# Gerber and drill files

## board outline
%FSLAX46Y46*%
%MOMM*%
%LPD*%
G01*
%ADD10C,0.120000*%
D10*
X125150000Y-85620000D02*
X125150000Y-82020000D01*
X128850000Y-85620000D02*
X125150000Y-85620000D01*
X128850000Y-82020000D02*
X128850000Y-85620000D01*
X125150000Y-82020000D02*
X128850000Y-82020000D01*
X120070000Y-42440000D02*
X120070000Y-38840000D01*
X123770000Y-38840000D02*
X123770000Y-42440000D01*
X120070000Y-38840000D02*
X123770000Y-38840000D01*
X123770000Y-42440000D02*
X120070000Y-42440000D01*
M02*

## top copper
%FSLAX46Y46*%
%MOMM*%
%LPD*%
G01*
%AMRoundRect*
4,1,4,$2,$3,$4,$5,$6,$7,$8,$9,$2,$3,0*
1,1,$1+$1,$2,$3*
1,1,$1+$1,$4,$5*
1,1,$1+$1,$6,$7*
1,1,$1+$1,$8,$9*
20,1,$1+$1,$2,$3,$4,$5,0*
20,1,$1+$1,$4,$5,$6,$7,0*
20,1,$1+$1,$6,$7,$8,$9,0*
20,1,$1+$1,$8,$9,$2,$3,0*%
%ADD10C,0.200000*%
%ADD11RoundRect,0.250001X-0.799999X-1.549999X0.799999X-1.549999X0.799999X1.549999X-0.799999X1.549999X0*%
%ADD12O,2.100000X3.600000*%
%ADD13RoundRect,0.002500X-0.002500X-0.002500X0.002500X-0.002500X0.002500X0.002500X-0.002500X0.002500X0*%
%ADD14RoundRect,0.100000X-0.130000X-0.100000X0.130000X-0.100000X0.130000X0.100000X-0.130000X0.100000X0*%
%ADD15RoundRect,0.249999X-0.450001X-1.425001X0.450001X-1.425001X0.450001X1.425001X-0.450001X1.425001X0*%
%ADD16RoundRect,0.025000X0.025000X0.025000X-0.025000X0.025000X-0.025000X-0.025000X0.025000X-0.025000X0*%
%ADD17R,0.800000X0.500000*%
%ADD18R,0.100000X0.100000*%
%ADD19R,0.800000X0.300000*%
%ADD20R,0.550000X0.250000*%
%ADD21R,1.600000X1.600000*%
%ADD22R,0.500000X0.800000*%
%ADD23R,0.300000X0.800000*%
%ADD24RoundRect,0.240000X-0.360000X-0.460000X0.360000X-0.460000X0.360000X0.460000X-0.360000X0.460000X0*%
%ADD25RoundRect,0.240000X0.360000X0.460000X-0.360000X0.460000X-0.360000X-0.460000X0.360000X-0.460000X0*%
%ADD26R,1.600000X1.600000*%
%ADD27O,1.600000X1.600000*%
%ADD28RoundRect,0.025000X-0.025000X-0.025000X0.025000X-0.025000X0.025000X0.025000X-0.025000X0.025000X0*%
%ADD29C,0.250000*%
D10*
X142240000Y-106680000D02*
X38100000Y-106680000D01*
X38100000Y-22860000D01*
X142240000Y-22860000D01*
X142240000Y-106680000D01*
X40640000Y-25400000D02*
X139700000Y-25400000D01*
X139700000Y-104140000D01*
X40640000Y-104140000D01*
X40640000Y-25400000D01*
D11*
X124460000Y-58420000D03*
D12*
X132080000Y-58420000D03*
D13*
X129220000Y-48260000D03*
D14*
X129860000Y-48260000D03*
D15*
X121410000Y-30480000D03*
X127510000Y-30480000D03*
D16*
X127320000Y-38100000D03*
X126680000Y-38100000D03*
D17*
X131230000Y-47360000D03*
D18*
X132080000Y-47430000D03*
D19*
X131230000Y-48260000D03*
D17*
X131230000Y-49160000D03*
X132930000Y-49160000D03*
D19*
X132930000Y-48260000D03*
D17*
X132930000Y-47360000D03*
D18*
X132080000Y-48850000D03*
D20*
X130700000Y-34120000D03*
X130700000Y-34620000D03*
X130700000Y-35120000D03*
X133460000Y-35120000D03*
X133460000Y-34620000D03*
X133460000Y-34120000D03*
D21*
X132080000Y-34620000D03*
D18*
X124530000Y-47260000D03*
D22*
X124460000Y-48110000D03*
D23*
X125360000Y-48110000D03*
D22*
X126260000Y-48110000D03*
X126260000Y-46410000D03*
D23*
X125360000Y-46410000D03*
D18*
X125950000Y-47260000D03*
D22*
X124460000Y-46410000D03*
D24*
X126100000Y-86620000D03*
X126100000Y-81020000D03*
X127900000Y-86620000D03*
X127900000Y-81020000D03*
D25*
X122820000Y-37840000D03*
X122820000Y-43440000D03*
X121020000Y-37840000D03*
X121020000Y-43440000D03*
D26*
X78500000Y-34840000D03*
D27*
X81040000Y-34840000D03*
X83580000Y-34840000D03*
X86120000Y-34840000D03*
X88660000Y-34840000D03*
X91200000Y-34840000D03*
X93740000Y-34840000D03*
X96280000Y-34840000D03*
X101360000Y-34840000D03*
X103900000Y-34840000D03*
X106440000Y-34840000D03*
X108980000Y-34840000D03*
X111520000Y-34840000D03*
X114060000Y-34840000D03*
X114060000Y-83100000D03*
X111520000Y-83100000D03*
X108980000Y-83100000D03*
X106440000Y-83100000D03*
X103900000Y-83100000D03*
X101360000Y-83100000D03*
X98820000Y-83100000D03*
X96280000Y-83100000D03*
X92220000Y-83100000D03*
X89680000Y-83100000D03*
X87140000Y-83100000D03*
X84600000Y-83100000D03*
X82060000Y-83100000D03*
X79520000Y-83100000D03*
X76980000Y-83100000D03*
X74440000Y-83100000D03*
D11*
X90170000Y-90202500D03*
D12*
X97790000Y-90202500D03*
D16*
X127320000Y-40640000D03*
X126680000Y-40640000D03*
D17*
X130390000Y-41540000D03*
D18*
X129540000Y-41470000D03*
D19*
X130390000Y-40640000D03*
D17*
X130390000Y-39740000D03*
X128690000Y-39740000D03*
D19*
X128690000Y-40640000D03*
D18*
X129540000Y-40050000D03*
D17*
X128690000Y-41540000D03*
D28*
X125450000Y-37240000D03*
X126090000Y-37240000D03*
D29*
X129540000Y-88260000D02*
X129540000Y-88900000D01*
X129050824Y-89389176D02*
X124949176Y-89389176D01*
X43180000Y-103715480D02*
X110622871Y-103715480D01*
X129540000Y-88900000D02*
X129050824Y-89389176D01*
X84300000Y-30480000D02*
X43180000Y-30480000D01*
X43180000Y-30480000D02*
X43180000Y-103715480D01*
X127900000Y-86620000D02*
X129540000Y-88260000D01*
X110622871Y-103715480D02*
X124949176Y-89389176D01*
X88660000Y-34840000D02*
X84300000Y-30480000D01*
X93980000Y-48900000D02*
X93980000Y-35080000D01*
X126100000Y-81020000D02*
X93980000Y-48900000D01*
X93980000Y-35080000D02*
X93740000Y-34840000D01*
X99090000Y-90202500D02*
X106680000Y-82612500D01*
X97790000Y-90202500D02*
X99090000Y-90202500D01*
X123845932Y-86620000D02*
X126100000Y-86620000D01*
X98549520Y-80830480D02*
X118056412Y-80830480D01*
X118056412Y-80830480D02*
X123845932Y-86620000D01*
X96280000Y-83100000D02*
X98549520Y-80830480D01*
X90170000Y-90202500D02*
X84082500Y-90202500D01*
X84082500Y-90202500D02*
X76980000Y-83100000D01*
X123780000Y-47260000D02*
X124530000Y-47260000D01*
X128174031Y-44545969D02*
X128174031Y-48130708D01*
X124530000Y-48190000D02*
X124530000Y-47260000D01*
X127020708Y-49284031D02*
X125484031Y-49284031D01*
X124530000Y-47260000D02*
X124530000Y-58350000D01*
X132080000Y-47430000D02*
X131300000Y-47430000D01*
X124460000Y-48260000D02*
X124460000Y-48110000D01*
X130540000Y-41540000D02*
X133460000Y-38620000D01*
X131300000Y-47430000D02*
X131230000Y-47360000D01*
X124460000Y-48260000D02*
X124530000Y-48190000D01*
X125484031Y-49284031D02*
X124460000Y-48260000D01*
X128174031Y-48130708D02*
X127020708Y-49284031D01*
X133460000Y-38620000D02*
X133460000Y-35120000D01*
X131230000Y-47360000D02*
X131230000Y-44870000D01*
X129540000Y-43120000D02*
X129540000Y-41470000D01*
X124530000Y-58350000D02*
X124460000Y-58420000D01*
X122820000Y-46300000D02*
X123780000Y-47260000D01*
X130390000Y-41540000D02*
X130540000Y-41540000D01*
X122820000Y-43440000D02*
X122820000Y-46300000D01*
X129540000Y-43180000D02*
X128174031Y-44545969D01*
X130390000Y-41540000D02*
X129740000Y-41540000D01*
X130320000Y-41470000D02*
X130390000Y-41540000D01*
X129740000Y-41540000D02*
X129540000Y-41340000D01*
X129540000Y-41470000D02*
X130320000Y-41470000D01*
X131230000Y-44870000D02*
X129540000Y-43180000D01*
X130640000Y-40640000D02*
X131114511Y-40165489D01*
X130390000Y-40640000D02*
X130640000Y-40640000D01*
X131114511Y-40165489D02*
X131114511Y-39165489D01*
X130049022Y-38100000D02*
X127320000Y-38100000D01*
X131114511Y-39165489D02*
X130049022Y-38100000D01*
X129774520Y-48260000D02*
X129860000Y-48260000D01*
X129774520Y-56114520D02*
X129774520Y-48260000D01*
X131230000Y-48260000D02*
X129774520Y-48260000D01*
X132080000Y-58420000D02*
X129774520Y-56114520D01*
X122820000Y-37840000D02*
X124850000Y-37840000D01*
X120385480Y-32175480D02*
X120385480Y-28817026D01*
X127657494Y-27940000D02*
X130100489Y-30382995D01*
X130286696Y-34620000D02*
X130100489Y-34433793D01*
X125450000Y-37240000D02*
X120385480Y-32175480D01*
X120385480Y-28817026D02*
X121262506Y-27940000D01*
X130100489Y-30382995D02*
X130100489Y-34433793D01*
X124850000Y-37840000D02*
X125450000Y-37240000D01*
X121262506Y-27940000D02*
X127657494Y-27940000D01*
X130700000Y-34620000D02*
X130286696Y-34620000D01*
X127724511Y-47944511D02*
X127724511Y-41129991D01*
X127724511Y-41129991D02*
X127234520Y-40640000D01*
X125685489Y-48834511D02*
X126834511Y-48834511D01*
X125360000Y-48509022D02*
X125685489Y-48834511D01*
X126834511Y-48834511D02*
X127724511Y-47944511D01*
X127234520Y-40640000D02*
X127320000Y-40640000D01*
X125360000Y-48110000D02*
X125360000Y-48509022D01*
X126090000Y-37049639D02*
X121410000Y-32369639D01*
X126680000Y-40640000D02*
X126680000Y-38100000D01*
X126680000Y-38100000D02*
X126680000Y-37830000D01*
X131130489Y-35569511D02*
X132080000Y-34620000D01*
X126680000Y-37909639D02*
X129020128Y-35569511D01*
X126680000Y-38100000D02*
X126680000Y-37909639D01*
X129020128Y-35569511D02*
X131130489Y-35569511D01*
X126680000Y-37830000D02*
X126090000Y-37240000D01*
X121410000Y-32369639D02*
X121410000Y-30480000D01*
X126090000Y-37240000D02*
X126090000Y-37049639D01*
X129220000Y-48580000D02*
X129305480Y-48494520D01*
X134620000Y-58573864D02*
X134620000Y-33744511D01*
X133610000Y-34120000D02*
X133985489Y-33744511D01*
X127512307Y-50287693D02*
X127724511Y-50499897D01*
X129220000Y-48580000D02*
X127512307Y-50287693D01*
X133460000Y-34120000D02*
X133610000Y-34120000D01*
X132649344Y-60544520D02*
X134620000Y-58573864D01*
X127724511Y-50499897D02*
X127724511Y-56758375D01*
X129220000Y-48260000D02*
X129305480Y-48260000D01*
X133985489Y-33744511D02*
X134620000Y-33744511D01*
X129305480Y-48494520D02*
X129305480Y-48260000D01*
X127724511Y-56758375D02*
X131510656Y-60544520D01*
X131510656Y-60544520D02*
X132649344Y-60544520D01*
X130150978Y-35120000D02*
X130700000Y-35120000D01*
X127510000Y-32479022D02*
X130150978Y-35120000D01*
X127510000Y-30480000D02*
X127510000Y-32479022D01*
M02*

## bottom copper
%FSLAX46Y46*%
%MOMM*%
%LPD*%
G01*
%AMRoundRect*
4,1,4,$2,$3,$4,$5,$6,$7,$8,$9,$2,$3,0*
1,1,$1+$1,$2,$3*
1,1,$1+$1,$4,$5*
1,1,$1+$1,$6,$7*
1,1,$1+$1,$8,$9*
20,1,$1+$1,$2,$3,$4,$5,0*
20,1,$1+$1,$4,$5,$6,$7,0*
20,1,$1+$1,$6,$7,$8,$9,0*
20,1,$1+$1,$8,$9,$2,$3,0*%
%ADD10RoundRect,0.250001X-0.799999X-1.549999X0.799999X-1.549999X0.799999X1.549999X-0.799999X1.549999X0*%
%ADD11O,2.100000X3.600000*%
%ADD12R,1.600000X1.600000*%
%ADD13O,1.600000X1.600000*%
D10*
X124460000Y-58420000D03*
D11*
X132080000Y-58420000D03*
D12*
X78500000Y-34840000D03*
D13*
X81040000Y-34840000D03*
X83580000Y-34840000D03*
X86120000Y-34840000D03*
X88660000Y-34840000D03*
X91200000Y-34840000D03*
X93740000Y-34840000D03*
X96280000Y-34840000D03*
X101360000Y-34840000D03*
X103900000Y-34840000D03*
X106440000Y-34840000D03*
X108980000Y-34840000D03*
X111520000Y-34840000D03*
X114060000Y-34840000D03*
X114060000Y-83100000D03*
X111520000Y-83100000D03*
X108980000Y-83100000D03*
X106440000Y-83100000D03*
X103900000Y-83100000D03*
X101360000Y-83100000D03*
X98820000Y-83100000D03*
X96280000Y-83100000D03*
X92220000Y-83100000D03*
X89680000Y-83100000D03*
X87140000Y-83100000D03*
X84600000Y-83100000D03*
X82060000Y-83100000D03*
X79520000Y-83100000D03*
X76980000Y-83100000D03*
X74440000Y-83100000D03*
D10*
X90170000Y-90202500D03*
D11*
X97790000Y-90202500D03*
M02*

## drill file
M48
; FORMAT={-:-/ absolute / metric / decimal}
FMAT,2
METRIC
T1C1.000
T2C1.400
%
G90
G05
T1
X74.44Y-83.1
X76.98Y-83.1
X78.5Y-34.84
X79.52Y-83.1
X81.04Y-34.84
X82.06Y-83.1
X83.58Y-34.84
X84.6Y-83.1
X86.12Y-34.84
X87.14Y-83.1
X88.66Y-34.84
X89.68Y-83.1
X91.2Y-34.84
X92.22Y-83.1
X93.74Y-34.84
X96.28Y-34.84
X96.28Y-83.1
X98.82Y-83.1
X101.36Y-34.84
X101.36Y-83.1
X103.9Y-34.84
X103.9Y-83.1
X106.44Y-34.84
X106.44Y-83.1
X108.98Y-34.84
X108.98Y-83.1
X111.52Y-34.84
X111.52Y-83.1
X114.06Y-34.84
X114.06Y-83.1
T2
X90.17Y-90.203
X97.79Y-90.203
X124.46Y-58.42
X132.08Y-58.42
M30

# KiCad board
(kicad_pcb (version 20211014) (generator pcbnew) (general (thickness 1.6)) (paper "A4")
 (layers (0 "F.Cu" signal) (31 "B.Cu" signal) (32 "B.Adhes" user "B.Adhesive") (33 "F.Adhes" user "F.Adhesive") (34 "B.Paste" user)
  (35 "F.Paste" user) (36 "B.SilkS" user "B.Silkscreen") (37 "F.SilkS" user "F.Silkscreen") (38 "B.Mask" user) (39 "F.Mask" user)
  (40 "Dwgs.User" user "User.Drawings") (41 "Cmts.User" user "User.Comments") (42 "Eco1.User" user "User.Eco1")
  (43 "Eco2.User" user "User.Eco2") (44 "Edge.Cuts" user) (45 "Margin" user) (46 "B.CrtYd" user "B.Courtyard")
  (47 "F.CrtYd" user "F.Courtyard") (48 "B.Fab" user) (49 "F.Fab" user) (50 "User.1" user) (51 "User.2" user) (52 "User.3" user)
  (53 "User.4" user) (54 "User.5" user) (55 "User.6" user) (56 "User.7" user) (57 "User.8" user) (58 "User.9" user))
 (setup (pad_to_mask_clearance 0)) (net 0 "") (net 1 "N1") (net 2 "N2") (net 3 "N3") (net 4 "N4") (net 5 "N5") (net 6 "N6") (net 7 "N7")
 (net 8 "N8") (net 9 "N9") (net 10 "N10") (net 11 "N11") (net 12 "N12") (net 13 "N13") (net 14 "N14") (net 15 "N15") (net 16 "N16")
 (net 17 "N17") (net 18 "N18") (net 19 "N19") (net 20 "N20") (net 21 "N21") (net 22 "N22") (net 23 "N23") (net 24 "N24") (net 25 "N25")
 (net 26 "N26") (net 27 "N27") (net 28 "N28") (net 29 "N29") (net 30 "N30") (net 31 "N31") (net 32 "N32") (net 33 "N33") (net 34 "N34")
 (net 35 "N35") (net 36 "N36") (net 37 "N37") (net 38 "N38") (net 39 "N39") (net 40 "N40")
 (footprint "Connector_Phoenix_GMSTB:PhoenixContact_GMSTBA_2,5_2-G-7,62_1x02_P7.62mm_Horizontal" (layer "F.Cu") (at 124.46 58.42)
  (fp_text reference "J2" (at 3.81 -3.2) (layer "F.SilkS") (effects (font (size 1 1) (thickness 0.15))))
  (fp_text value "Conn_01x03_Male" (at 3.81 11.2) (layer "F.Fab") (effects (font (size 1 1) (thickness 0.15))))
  (pad "1" thru_hole roundrect (at 0 0) (size 2.1 3.6) (drill 1.4) (layers *.Cu *.Mask) (roundrect_rratio 0.119048) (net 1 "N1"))
  (pad "2" thru_hole oval (at 7.62 0) (size 2.1 3.6) (drill 1.4) (layers *.Cu *.Mask) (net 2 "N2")))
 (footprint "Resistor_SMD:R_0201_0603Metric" (layer "F.Cu") (at 129.54 48.26)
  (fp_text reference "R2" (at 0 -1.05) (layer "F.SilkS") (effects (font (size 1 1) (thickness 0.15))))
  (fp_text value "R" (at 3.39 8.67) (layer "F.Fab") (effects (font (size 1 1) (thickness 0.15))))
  (pad "" smd roundrect (at -0.345 0) (size 0.318 0.36) (layers "F.Paste") (roundrect_rratio 0.25))
  (pad "" smd roundrect (at 0.345 0) (size 0.318 0.36) (layers "F.Paste") (roundrect_rratio 0.25))
  (pad "1" smd roundrect (at -0.32 0) (size 0.01 0.01) (layers "F.Cu" "F.Mask") (roundrect_rratio 0.25) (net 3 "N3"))
  (pad "2" smd roundrect (at 0.32 0) (size 0.46 0.4) (layers "F.Cu" "F.Mask") (roundrect_rratio 0.25) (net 2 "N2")))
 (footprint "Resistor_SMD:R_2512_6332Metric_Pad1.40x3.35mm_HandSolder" (layer "F.Cu") (at 124.46 30.48)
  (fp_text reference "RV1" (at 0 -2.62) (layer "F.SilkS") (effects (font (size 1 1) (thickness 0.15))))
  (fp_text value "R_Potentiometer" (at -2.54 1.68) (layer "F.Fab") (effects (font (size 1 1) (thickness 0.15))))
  (pad "1" smd roundrect (at -3.05 0) (size 1.4 3.35) (layers "F.Cu" "F.Paste" "F.Mask") (roundrect_rratio 0.178571) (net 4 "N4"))
  (pad "2" smd roundrect (at 3.05 0) (size 1.4 3.35) (layers "F.Cu" "F.Paste" "F.Mask") (roundrect_rratio 0.178571) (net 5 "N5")))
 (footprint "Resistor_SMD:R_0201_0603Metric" (layer "F.Cu") (at 127 38.1 180)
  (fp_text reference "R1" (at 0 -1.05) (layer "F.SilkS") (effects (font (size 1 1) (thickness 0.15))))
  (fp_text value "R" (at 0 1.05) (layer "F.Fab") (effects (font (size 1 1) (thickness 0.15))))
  (pad "" smd roundrect (at -0.345 0 180) (size 0.318 0.36) (layers "F.Paste") (roundrect_rratio 0.25))
  (pad "" smd roundrect (at 0.345 0 180) (size 0.1 0.1) (layers "F.Paste") (roundrect_rratio 0.25))
  (pad "1" smd roundrect (at -0.32 0 180) (size 0.1 0.1) (layers "F.Cu" "F.Mask") (roundrect_rratio 0.25) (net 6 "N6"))
  (pad "2" smd roundrect (at 0.32 0 180) (size 0.1 0.1) (layers "F.Cu" "F.Mask") (roundrect_rratio 0.25) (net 4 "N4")))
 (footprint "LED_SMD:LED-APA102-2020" (layer "F.Cu") (at 132.08 48.26)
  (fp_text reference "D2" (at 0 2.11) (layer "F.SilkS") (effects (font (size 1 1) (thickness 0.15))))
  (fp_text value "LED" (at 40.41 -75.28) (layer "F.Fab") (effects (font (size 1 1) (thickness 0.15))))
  (pad "1" smd rect (at -0.85 -0.9) (size 0.8 0.5) (layers "F.Cu" "F.Paste" "F.Mask") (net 1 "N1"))
  (pad "1" smd rect (at 0 -0.83 90) (size 0.1 0.1) (layers "F.Cu" "F.Paste" "F.Mask") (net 1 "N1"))
  (pad "2" smd rect (at -0.85 0) (size 0.8 0.3) (layers "F.Cu" "F.Paste" "F.Mask") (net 2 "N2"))
  (pad "3" smd rect (at -0.85 0.9) (size 0.8 0.5) (layers "F.Cu" "F.Paste" "F.Mask"))
  (pad "4" smd rect (at 0.85 0.9) (size 0.8 0.5) (layers "F.Cu" "F.Paste" "F.Mask"))
  (pad "5" smd rect (at 0.85 0) (size 0.8 0.3) (layers "F.Cu" "F.Paste" "F.Mask"))
  (pad "6" smd rect (at 0.85 -0.9) (size 0.8 0.5) (layers "F.Cu" "F.Paste" "F.Mask"))
  (pad "6" smd rect (at 0 0.59 90) (size 0.1 0.1) (layers "F.Cu" "F.Paste" "F.Mask")))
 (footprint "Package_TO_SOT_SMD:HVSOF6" (layer "F.Cu") (at 132.08 34.62)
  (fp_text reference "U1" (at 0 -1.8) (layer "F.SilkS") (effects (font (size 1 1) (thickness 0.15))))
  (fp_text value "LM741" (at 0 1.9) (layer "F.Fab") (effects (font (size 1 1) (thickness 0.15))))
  (pad "1" smd rect (at -1.38 -0.5 270) (size 0.25 0.55) (layers "F.Cu" "F.Paste" "F.Mask") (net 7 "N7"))
  (pad "2" smd rect (at -1.38 0 270) (size 0.25 0.55) (layers "F.Cu" "F.Paste" "F.Mask") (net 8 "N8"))
  (pad "3" smd rect (at -1.38 0.5 270) (size 0.25 0.55) (layers "F.Cu" "F.Paste" "F.Mask") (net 5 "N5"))
  (pad "4" smd rect (at 1.38 0.5 270) (size 0.25 0.55) (layers "F.Cu" "F.Paste" "F.Mask") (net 1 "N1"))
  (pad "5" smd rect (at 1.38 0 270) (size 0.25 0.55) (layers "F.Cu" "F.Paste" "F.Mask") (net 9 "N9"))
  (pad "6" smd rect (at 1.38 -0.5 270) (size 0.25 0.55) (layers "F.Cu" "F.Paste" "F.Mask") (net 3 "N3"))
  (pad "7" smd rect (at 0 0) (size 1.6 1.6) (layers "F.Cu" "F.Paste" "F.Mask") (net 4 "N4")))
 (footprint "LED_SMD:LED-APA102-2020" (layer "F.Cu") (at 125.36 47.26 90)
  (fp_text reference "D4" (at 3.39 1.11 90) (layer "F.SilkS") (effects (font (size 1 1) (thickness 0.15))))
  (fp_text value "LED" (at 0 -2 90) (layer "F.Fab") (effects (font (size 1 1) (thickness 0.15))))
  (pad "1" smd rect (at 0 -0.83 180) (size 0.1 0.1) (layers "F.Cu" "F.Paste" "F.Mask") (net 1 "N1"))
  (pad "1" smd rect (at -0.85 -0.9 90) (size 0.8 0.5) (layers "F.Cu" "F.Paste" "F.Mask") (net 1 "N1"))
  (pad "2" smd rect (at -0.85 0 90) (size 0.8 0.3) (layers "F.Cu" "F.Paste" "F.Mask") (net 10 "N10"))
  (pad "3" smd rect (at -0.85 0.9 90) (size 0.8 0.5) (layers "F.Cu" "F.Paste" "F.Mask"))
  (pad "4" smd rect (at 0.85 0.9 90) (size 0.8 0.5) (layers "F.Cu" "F.Paste" "F.Mask"))
  (pad "5" smd rect (at 0.85 0 90) (size 0.8 0.3) (layers "F.Cu" "F.Paste" "F.Mask"))
  (pad "6" smd rect (at 0 0.59 180) (size 0.1 0.1) (layers "F.Cu" "F.Paste" "F.Mask"))
  (pad "6" smd rect (at 0.85 -0.9 90) (size 0.8 0.5) (layers "F.Cu" "F.Paste" "F.Mask")))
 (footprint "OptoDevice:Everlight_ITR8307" (layer "F.Cu") (at 127 83.82)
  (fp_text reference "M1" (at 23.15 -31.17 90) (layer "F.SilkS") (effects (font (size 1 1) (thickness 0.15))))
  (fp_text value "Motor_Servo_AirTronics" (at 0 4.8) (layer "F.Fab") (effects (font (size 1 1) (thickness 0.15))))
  (fp_line (start -1.85 1.8) (end -1.85 -1.8) (layer "Edge.Cuts") (width 0.12))
  (fp_line (start 1.85 1.8) (end -1.85 1.8) (layer "Edge.Cuts") (width 0.12))
  (fp_line (start 1.85 -1.8) (end 1.85 1.8) (layer "Edge.Cuts") (width 0.12))
  (fp_line (start -1.85 -1.8) (end 1.85 -1.8) (layer "Edge.Cuts") (width 0.12))
  (pad "1" smd roundrect (at -0.9 2.8) (size 1.2 1.4) (layers "F.Cu" "F.Paste" "F.Mask") (roundrect_rratio 0.2) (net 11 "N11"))
  (pad "2" smd roundrect (at -0.9 -2.8) (size 1.2 1.4) (layers "F.Cu" "F.Paste" "F.Mask") (roundrect_rratio 0.2) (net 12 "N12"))
  (pad "3" smd roundrect (at 0.9 2.8) (size 1.2 1.4) (layers "F.Cu" "F.Paste" "F.Mask") (roundrect_rratio 0.2) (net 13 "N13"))
  (pad "4" smd roundrect (at 0.9 -2.8) (size 1.2 1.4) (layers "F.Cu" "F.Paste" "F.Mask") (roundrect_rratio 0.2)))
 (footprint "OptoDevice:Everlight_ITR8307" (layer "F.Cu") (at 121.92 40.64 180)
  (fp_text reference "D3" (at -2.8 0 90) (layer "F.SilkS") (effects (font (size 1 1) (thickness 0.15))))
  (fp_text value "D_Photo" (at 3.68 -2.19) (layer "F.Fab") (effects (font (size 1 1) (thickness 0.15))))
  (fp_line (start 1.85 -1.8) (end 1.85 1.8) (layer "Edge.Cuts") (width 0.12))
  (fp_line (start -1.85 1.8) (end -1.85 -1.8) (layer "Edge.Cuts") (width 0.12))
  (fp_line (start 1.85 1.8) (end -1.85 1.8) (layer "Edge.Cuts") (width 0.12))
  (fp_line (start -1.85 -1.8) (end 1.85 -1.8) (layer "Edge.Cuts") (width 0.12))
  (pad "1" smd roundrect (at -0.9 2.8 180) (size 1.2 1.4) (layers "F.Cu" "F.Paste" "F.Mask") (roundrect_rratio 0.2) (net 8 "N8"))
  (pad "2" smd roundrect (at -0.9 -2.8 180) (size 1.2 1.4) (layers "F.Cu" "F.Paste" "F.Mask") (roundrect_rratio 0.2) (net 1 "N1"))
  (pad "3" smd roundrect (at 0.9 2.8 180) (size 1.2 1.4) (layers "F.Cu" "F.Paste" "F.Mask") (roundrect_rratio 0.2))
  (pad "4" smd roundrect (at 0.9 -2.8 180) (size 1.2 1.4) (layers "F.Cu" "F.Paste" "F.Mask") (roundrect_rratio 0.2)))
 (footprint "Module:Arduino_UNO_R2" (layer "F.Cu") (at 78.5 34.84)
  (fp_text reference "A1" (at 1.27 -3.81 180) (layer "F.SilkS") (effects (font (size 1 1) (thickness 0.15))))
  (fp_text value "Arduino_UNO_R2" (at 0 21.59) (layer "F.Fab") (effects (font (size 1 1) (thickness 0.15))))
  (pad "1" thru_hole rect (at 0 0 90) (size 1.6 1.6) (drill 1) (layers *.Cu *.Mask) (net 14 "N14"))
  (pad "2" thru_hole oval (at 2.54 0 90) (size 1.6 1.6) (drill 1) (layers *.Cu *.Mask) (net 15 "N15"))
  (pad "3" thru_hole oval (at 5.08 0 90) (size 1.6 1.6) (drill 1) (layers *.Cu *.Mask) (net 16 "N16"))
  (pad "4" thru_hole oval (at 7.62 0 90) (size 1.6 1.6) (drill 1) (layers *.Cu *.Mask) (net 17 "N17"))
  (pad "5" thru_hole oval (at 10.16 0 90) (size 1.6 1.6) (drill 1) (layers *.Cu *.Mask) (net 13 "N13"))
  (pad "6" thru_hole oval (at 12.7 0 90) (size 1.6 1.6) (drill 1) (layers *.Cu *.Mask) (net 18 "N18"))
  (pad "7" thru_hole oval (at 15.24 0 90) (size 1.6 1.6) (drill 1) (layers *.Cu *.Mask) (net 12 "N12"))
  (pad "8" thru_hole oval (at 17.78 0 90) (size 1.6 1.6) (drill 1) (layers *.Cu *.Mask) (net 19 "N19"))
  (pad "9" thru_hole oval (at 22.86 0 90) (size 1.6 1.6) (drill 1) (layers *.Cu *.Mask) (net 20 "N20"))
  (pad "10" thru_hole oval (at 25.4 0 90) (size 1.6 1.6) (drill 1) (layers *.Cu *.Mask) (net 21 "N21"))
  (pad "11" thru_hole oval (at 27.94 0 90) (size 1.6 1.6) (drill 1) (layers *.Cu *.Mask) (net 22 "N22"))
  (pad "12" thru_hole oval (at 30.48 0 90) (size 1.6 1.6) (drill 1) (layers *.Cu *.Mask) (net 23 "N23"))
  (pad "13" thru_hole oval (at 33.02 0 90) (size 1.6 1.6) (drill 1) (layers *.Cu *.Mask) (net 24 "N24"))
  (pad "14" thru_hole oval (at 35.56 0 90) (size 1.6 1.6) (drill 1) (layers *.Cu *.Mask) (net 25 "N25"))
  (pad "15" thru_hole oval (at 35.56 48.26 90) (size 1.6 1.6) (drill 1) (layers *.Cu *.Mask) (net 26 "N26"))
  (pad "16" thru_hole oval (at 33.02 48.26 90) (size 1.6 1.6) (drill 1) (layers *.Cu *.Mask) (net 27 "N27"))
  (pad "17" thru_hole oval (at 30.48 48.26 90) (size 1.6 1.6) (drill 1) (layers *.Cu *.Mask) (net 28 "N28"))
  (pad "18" thru_hole oval (at 27.94 48.26 90) (size 1.6 1.6) (drill 1) (layers *.Cu *.Mask) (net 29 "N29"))
  (pad "19" thru_hole oval (at 25.4 48.26 90) (size 1.6 1.6) (drill 1) (layers *.Cu *.Mask) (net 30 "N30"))
  (pad "20" thru_hole oval (at 22.86 48.26 90) (size 1.6 1.6) (drill 1) (layers *.Cu *.Mask) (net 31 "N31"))
  (pad "21" thru_hole oval (at 20.32 48.26 90) (size 1.6 1.6) (drill 1) (layers *.Cu *.Mask) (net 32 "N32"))
  (pad "22" thru_hole oval (at 17.78 48.26 90) (size 1.6 1.6) (drill 1) (layers *.Cu *.Mask) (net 11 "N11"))
  (pad "23" thru_hole oval (at 13.72 48.26 90) (size 1.6 1.6) (drill 1) (layers *.Cu *.Mask) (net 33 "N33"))
  (pad "24" thru_hole oval (at 11.18 48.26 90) (size 1.6 1.6) (drill 1) (layers *.Cu *.Mask) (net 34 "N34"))
  (pad "25" thru_hole oval (at 8.64 48.26 90) (size 1.6 1.6) (drill 1) (layers *.Cu *.Mask) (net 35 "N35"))
  (pad "26" thru_hole oval (at 6.1 48.26 90) (size 1.6 1.6) (drill 1) (layers *.Cu *.Mask) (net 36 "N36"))
  (pad "27" thru_hole oval (at 3.56 48.26 90) (size 1.6 1.6) (drill 1) (layers *.Cu *.Mask) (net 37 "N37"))
  (pad "28" thru_hole oval (at 1.02 48.26 90) (size 1.6 1.6) (drill 1) (layers *.Cu *.Mask) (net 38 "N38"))
  (pad "29" thru_hole oval (at -1.52 48.26 90) (size 1.6 1.6) (drill 1) (layers *.Cu *.Mask) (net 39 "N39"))
  (pad "30" thru_hole oval (at -4.06 48.26 90) (size 1.6 1.6) (drill 1) (layers *.Cu *.Mask) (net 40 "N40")))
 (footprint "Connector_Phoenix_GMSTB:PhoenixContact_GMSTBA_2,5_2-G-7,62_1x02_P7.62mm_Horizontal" (layer "F.Cu") (at 90.17 90.2025)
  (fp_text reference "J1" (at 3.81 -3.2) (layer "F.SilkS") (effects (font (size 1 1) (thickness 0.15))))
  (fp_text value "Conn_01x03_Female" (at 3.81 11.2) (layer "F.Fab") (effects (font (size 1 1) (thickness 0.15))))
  (pad "1" thru_hole roundrect (at 0 0) (size 2.1 3.6) (drill 1.4) (layers *.Cu *.Mask) (roundrect_rratio 0.119048) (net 39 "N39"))
  (pad "2" thru_hole oval (at 7.62 0) (size 2.1 3.6) (drill 1.4) (layers *.Cu *.Mask) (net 29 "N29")))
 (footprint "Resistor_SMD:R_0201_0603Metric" (layer "F.Cu") (at 127 40.64 180)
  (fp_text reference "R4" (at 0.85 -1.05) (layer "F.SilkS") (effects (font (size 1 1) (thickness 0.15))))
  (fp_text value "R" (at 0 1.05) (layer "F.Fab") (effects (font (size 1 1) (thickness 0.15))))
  (pad "" smd roundrect (at 0.345 0 180) (size 0.318 0.36) (layers "F.Paste") (roundrect_rratio 0.25))
  (pad "" smd roundrect (at -0.345 0 180) (size 0.1 0.1) (layers "F.Paste") (roundrect_rratio 0.25))
  (pad "1" smd roundrect (at -0.32 0 180) (size 0.1 0.1) (layers "F.Cu" "F.Mask") (roundrect_rratio 0.25) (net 10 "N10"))
  (pad "2" smd roundrect (at 0.32 0 180) (size 0.1 0.1) (layers "F.Cu" "F.Mask") (roundrect_rratio 0.25) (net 4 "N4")))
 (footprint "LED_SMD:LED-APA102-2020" (layer "F.Cu") (at 129.54 40.64 180)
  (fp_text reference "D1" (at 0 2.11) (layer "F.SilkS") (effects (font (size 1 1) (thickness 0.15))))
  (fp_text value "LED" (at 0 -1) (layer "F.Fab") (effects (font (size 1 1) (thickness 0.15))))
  (pad "1" smd rect (at -0.85 -0.9 180) (size 0.8 0.5) (layers "F.Cu" "F.Paste" "F.Mask") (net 1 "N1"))
  (pad "1" smd rect (at 0 -0.83 270) (size 0.1 0.1) (layers "F.Cu" "F.Paste" "F.Mask") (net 1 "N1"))
  (pad "2" smd rect (at -0.85 0 180) (size 0.8 0.3) (layers "F.Cu" "F.Paste" "F.Mask") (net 6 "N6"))
  (pad "3" smd rect (at -0.85 0.9 180) (size 0.8 0.5) (layers "F.Cu" "F.Paste" "F.Mask"))
  (pad "4" smd rect (at 0.85 0.9 180) (size 0.8 0.5) (layers "F.Cu" "F.Paste" "F.Mask"))
  (pad "5" smd rect (at 0.85 0 180) (size 0.8 0.3) (layers "F.Cu" "F.Paste" "F.Mask"))
  (pad "6" smd rect (at 0 0.59 270) (size 0.1 0.1) (layers "F.Cu" "F.Paste" "F.Mask"))
  (pad "6" smd rect (at 0.85 -0.9 180) (size 0.8 0.5) (layers "F.Cu" "F.Paste" "F.Mask")))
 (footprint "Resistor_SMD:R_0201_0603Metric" (layer "F.Cu") (at 125.77 37.24)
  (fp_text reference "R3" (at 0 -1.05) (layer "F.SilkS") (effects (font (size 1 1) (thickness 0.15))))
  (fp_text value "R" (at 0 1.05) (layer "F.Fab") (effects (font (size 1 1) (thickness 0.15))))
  (pad "" smd roundrect (at -0.345 0) (size 0.318 0.36) (layers "F.Paste") (roundrect_rratio 0.25))
  (pad "" smd roundrect (at 0.345 0) (size 0.318 0.36) (layers "F.Paste") (roundrect_rratio 0.25))
  (pad "1" smd roundrect (at -0.32 0) (size 0.1 0.1) (layers "F.Cu" "F.Mask") (roundrect_rratio 0.25) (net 8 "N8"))
  (pad "2" smd roundrect (at 0.32 0) (size 0.1 0.1) (layers "F.Cu" "F.Mask") (roundrect_rratio 0.25) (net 4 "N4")))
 (gr_poly (pts (xy 142.24 106.68) (xy 38.1 106.68) (xy 38.1 22.86) (xy 142.24 22.86)) (layer "F.Cu") (width 0.2) (fill none))
 (gr_rect locked (start 40.64 25.4) (end 139.7 104.14) (layer "F.Cu") (width 0.2) (fill none))
 (segment (start 129.54 88.26) (end 129.54 88.9) (width 0.25) (layer "F.Cu") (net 13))
 (segment (start 129.050824 89.389176) (end 124.949176 89.389176) (width 0.25) (layer "F.Cu") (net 13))
 (segment (start 43.18 103.71548) (end 110.622871 103.71548) (width 0.25) (layer "F.Cu") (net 13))
 (segment (start 129.54 88.9) (end 129.050824 89.389176) (width 0.25) (layer "F.Cu") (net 13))
 (segment (start 84.3 30.48) (end 43.18 30.48) (width 0.25) (layer "F.Cu") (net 13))
 (segment (start 43.18 30.48) (end 43.18 103.71548) (width 0.25) (layer "F.Cu") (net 13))
 (segment (start 127.9 86.62) (end 129.54 88.26) (width 0.25) (layer "F.Cu") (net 13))
 (segment (start 110.622871 103.71548) (end 124.949176 89.389176) (width 0.25) (layer "F.Cu") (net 13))
 (segment (start 88.66 34.84) (end 84.3 30.48) (width 0.25) (layer "F.Cu") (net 13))
 (segment (start 93.98 48.9) (end 93.98 35.08) (width 0.25) (layer "F.Cu") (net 12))
 (segment (start 126.1 81.02) (end 93.98 48.9) (width 0.25) (layer "F.Cu") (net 12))
 (segment (start 93.98 35.08) (end 93.74 34.84) (width 0.25) (layer "F.Cu") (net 12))
 (segment (start 99.09 90.2025) (end 106.68 82.6125) (width 0.25) (layer "F.Cu") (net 29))
 (segment (start 97.79 90.2025) (end 99.09 90.2025) (width 0.25) (layer "F.Cu") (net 29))
 (segment (start 123.845932 86.62) (end 126.1 86.62) (width 0.25) (layer "F.Cu") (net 11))
 (segment (start 98.54952 80.83048) (end 118.056412 80.83048) (width 0.25) (layer "F.Cu") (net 11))
 (segment (start 118.056412 80.83048) (end 123.845932 86.62) (width 0.25) (layer "F.Cu") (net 11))
 (segment (start 96.28 83.1) (end 98.54952 80.83048) (width 0.25) (layer "F.Cu") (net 11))
 (segment (start 90.17 90.2025) (end 84.0825 90.2025) (width 0.25) (layer "F.Cu") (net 39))
 (segment (start 84.0825 90.2025) (end 76.98 83.1) (width 0.25) (layer "F.Cu") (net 39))
 (segment (start 123.78 47.26) (end 124.53 47.26) (width 0.25) (layer "F.Cu") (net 1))
 (segment (start 128.174031 44.545969) (end 128.174031 48.130708) (width 0.25) (layer "F.Cu") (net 1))
 (segment (start 124.53 48.19) (end 124.53 47.26) (width 0.25) (layer "F.Cu") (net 1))
 (segment (start 127.020708 49.284031) (end 125.484031 49.284031) (width 0.25) (layer "F.Cu") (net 1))
 (segment (start 124.53 47.26) (end 124.53 58.35) (width 0.25) (layer "F.Cu") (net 1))
 (segment (start 132.08 47.43) (end 131.3 47.43) (width 0.25) (layer "F.Cu") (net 1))
 (segment (start 124.46 48.26) (end 124.46 48.11) (width 0.25) (layer "F.Cu") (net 1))
 (segment (start 130.54 41.54) (end 133.46 38.62) (width 0.25) (layer "F.Cu") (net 1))
 (segment (start 131.3 47.43) (end 131.23 47.36) (width 0.25) (layer "F.Cu") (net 1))
 (segment (start 124.46 48.26) (end 124.53 48.19) (width 0.25) (layer "F.Cu") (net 1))
 (segment (start 125.484031 49.284031) (end 124.46 48.26) (width 0.25) (layer "F.Cu") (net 1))
 (segment (start 128.174031 48.130708) (end 127.020708 49.284031) (width 0.25) (layer "F.Cu") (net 1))
 (segment (start 133.46 38.62) (end 133.46 35.12) (width 0.25) (layer "F.Cu") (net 1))
 (segment (start 131.23 47.36) (end 131.23 44.87) (width 0.25) (layer "F.Cu") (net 1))
 (segment (start 129.54 43.12) (end 129.54 41.47) (width 0.25) (layer "F.Cu") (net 1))
 (segment (start 124.53 58.35) (end 124.46 58.42) (width 0.25) (layer "F.Cu") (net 1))
 (segment (start 122.82 46.3) (end 123.78 47.26) (width 0.25) (layer "F.Cu") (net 1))
 (segment (start 130.39 41.54) (end 130.54 41.54) (width 0.25) (layer "F.Cu") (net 1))
 (segment (start 122.82 43.44) (end 122.82 46.3) (width 0.25) (layer "F.Cu") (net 1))
 (segment (start 129.54 43.18) (end 128.174031 44.545969) (width 0.25) (layer "F.Cu") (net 1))
 (segment (start 130.39 41.54) (end 129.74 41.54) (width 0.25) (layer "F.Cu") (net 1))
 (segment (start 130.32 41.47) (end 130.39 41.54) (width 0.25) (layer "F.Cu") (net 1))
 (segment (start 129.74 41.54) (end 129.54 41.34) (width 0.25) (layer "F.Cu") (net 1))
 (segment (start 129.54 41.47) (end 130.32 41.47) (width 0.25) (layer "F.Cu") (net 1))
 (segment (start 131.23 44.87) (end 129.54 43.18) (width 0.25) (layer "F.Cu") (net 1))
 (segment (start 130.64 40.64) (end 131.114511 40.165489) (width 0.25) (layer "F.Cu") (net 6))
 (segment (start 130.39 40.64) (end 130.64 40.64) (width 0.25) (layer "F.Cu") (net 6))
 (segment (start 131.114511 40.165489) (end 131.114511 39.165489) (width 0.25) (layer "F.Cu") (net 6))
 (segment (start 130.049022 38.1) (end 127.32 38.1) (width 0.25) (layer "F.Cu") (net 6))
 (segment (start 131.114511 39.165489) (end 130.049022 38.1) (width 0.25) (layer "F.Cu") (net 6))
 (segment (start 129.77452 48.26) (end 129.86 48.26) (width 0.25) (layer "F.Cu") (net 2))
 (segment (start 129.77452 56.11452) (end 129.77452 48.26) (width 0.25) (layer "F.Cu") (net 2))
 (segment (start 131.23 48.26) (end 129.77452 48.26) (width 0.25) (layer "F.Cu") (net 2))
 (segment (start 132.08 58.42) (end 129.77452 56.11452) (width 0.25) (layer "F.Cu") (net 2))
 (segment (start 122.82 37.84) (end 124.85 37.84) (width 0.25) (layer "F.Cu") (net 8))
 (segment (start 120.38548 32.17548) (end 120.38548 28.817026) (width 0.25) (layer "F.Cu") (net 8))
 (segment (start 127.657494 27.94) (end 130.100489 30.382995) (width 0.25) (layer "F.Cu") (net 8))
 (segment (start 130.286696 34.62) (end 130.100489 34.433793) (width 0.25) (layer "F.Cu") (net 8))
 (segment (start 125.45 37.24) (end 120.38548 32.17548) (width 0.25) (layer "F.Cu") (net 8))
 (segment (start 120.38548 28.817026) (end 121.262506 27.94) (width 0.25) (layer "F.Cu") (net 8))
 (segment (start 130.100489 30.382995) (end 130.100489 34.433793) (width 0.25) (layer "F.Cu") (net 8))
 (segment (start 124.85 37.84) (end 125.45 37.24) (width 0.25) (layer "F.Cu") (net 8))
 (segment (start 121.262506 27.94) (end 127.657494 27.94) (width 0.25) (layer "F.Cu") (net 8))
 (segment (start 130.7 34.62) (end 130.286696 34.62) (width 0.25) (layer "F.Cu") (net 8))
 (segment (start 127.724511 47.944511) (end 127.724511 41.129991) (width 0.25) (layer "F.Cu") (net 10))
 (segment (start 127.724511 41.129991) (end 127.23452 40.64) (width 0.25) (layer "F.Cu") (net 10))
 (segment (start 125.685489 48.834511) (end 126.834511 48.834511) (width 0.25) (layer "F.Cu") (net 10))
 (segment (start 125.36 48.509022) (end 125.685489 48.834511) (width 0.25) (layer "F.Cu") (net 10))
 (segment (start 126.834511 48.834511) (end 127.724511 47.944511) (width 0.25) (layer "F.Cu") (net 10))
 (segment (start 127.23452 40.64) (end 127.32 40.64) (width 0.25) (layer "F.Cu") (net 10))
 (segment (start 125.36 48.11) (end 125.36 48.509022) (width 0.25) (layer "F.Cu") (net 10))
 (segment (start 126.09 37.049639) (end 121.41 32.369639) (width 0.25) (layer "F.Cu") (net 4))
 (segment (start 126.68 40.64) (end 126.68 38.1) (width 0.25) (layer "F.Cu") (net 4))
 (segment (start 126.68 38.1) (end 126.68 37.83) (width 0.25) (layer "F.Cu") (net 4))
 (segment (start 131.130489 35.569511) (end 132.08 34.62) (width 0.25) (layer "F.Cu") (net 4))
 (segment (start 126.68 37.909639) (end 129.020128 35.569511) (width 0.25) (layer "F.Cu") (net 4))
 (segment (start 126.68 38.1) (end 126.68 37.909639) (width 0.25) (layer "F.Cu") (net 4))
 (segment (start 129.020128 35.569511) (end 131.130489 35.569511) (width 0.25) (layer "F.Cu") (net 4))
 (segment (start 126.68 37.83) (end 126.09 37.24) (width 0.25) (layer "F.Cu") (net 4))
 (segment (start 121.41 32.369639) (end 121.41 30.48) (width 0.25) (layer "F.Cu") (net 4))
 (segment (start 126.09 37.24) (end 126.09 37.049639) (width 0.25) (layer "F.Cu") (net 4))
 (segment (start 129.22 48.58) (end 129.30548 48.49452) (width 0.25) (layer "F.Cu") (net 3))
 (segment (start 134.62 58.573864) (end 134.62 33.744511) (width 0.25) (layer "F.Cu") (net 3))
 (segment (start 133.61 34.12) (end 133.985489 33.744511) (width 0.25) (layer "F.Cu") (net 3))
 (segment (start 127.512307 50.287693) (end 127.724511 50.499897) (width 0.25) (layer "F.Cu") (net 3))
 (segment (start 129.22 48.58) (end 127.512307 50.287693) (width 0.25) (layer "F.Cu") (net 3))
 (segment (start 133.46 34.12) (end 133.61 34.12) (width 0.25) (layer "F.Cu") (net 3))
 (segment (start 132.649344 60.54452) (end 134.62 58.573864) (width 0.25) (layer "F.Cu") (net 3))
 (segment (start 127.724511 50.499897) (end 127.724511 56.758375) (width 0.25) (layer "F.Cu") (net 3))
 (segment (start 129.22 48.26) (end 129.30548 48.26) (width 0.25) (layer "F.Cu") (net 3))
 (segment (start 133.985489 33.744511) (end 134.62 33.744511) (width 0.25) (layer "F.Cu") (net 3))
 (segment (start 129.30548 48.49452) (end 129.30548 48.26) (width 0.25) (layer "F.Cu") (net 3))
 (segment (start 127.724511 56.758375) (end 131.510656 60.54452) (width 0.25) (layer "F.Cu") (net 3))
 (segment (start 131.510656 60.54452) (end 132.649344 60.54452) (width 0.25) (layer "F.Cu") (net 3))
 (segment (start 130.150978 35.12) (end 130.7 35.12) (width 0.25) (layer "F.Cu") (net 5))
 (segment (start 127.51 32.479022) (end 130.150978 35.12) (width 0.25) (layer "F.Cu") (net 5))
 (segment (start 127.51 30.48) (end 127.51 32.479022) (width 0.25) (layer "F.Cu") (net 5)))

